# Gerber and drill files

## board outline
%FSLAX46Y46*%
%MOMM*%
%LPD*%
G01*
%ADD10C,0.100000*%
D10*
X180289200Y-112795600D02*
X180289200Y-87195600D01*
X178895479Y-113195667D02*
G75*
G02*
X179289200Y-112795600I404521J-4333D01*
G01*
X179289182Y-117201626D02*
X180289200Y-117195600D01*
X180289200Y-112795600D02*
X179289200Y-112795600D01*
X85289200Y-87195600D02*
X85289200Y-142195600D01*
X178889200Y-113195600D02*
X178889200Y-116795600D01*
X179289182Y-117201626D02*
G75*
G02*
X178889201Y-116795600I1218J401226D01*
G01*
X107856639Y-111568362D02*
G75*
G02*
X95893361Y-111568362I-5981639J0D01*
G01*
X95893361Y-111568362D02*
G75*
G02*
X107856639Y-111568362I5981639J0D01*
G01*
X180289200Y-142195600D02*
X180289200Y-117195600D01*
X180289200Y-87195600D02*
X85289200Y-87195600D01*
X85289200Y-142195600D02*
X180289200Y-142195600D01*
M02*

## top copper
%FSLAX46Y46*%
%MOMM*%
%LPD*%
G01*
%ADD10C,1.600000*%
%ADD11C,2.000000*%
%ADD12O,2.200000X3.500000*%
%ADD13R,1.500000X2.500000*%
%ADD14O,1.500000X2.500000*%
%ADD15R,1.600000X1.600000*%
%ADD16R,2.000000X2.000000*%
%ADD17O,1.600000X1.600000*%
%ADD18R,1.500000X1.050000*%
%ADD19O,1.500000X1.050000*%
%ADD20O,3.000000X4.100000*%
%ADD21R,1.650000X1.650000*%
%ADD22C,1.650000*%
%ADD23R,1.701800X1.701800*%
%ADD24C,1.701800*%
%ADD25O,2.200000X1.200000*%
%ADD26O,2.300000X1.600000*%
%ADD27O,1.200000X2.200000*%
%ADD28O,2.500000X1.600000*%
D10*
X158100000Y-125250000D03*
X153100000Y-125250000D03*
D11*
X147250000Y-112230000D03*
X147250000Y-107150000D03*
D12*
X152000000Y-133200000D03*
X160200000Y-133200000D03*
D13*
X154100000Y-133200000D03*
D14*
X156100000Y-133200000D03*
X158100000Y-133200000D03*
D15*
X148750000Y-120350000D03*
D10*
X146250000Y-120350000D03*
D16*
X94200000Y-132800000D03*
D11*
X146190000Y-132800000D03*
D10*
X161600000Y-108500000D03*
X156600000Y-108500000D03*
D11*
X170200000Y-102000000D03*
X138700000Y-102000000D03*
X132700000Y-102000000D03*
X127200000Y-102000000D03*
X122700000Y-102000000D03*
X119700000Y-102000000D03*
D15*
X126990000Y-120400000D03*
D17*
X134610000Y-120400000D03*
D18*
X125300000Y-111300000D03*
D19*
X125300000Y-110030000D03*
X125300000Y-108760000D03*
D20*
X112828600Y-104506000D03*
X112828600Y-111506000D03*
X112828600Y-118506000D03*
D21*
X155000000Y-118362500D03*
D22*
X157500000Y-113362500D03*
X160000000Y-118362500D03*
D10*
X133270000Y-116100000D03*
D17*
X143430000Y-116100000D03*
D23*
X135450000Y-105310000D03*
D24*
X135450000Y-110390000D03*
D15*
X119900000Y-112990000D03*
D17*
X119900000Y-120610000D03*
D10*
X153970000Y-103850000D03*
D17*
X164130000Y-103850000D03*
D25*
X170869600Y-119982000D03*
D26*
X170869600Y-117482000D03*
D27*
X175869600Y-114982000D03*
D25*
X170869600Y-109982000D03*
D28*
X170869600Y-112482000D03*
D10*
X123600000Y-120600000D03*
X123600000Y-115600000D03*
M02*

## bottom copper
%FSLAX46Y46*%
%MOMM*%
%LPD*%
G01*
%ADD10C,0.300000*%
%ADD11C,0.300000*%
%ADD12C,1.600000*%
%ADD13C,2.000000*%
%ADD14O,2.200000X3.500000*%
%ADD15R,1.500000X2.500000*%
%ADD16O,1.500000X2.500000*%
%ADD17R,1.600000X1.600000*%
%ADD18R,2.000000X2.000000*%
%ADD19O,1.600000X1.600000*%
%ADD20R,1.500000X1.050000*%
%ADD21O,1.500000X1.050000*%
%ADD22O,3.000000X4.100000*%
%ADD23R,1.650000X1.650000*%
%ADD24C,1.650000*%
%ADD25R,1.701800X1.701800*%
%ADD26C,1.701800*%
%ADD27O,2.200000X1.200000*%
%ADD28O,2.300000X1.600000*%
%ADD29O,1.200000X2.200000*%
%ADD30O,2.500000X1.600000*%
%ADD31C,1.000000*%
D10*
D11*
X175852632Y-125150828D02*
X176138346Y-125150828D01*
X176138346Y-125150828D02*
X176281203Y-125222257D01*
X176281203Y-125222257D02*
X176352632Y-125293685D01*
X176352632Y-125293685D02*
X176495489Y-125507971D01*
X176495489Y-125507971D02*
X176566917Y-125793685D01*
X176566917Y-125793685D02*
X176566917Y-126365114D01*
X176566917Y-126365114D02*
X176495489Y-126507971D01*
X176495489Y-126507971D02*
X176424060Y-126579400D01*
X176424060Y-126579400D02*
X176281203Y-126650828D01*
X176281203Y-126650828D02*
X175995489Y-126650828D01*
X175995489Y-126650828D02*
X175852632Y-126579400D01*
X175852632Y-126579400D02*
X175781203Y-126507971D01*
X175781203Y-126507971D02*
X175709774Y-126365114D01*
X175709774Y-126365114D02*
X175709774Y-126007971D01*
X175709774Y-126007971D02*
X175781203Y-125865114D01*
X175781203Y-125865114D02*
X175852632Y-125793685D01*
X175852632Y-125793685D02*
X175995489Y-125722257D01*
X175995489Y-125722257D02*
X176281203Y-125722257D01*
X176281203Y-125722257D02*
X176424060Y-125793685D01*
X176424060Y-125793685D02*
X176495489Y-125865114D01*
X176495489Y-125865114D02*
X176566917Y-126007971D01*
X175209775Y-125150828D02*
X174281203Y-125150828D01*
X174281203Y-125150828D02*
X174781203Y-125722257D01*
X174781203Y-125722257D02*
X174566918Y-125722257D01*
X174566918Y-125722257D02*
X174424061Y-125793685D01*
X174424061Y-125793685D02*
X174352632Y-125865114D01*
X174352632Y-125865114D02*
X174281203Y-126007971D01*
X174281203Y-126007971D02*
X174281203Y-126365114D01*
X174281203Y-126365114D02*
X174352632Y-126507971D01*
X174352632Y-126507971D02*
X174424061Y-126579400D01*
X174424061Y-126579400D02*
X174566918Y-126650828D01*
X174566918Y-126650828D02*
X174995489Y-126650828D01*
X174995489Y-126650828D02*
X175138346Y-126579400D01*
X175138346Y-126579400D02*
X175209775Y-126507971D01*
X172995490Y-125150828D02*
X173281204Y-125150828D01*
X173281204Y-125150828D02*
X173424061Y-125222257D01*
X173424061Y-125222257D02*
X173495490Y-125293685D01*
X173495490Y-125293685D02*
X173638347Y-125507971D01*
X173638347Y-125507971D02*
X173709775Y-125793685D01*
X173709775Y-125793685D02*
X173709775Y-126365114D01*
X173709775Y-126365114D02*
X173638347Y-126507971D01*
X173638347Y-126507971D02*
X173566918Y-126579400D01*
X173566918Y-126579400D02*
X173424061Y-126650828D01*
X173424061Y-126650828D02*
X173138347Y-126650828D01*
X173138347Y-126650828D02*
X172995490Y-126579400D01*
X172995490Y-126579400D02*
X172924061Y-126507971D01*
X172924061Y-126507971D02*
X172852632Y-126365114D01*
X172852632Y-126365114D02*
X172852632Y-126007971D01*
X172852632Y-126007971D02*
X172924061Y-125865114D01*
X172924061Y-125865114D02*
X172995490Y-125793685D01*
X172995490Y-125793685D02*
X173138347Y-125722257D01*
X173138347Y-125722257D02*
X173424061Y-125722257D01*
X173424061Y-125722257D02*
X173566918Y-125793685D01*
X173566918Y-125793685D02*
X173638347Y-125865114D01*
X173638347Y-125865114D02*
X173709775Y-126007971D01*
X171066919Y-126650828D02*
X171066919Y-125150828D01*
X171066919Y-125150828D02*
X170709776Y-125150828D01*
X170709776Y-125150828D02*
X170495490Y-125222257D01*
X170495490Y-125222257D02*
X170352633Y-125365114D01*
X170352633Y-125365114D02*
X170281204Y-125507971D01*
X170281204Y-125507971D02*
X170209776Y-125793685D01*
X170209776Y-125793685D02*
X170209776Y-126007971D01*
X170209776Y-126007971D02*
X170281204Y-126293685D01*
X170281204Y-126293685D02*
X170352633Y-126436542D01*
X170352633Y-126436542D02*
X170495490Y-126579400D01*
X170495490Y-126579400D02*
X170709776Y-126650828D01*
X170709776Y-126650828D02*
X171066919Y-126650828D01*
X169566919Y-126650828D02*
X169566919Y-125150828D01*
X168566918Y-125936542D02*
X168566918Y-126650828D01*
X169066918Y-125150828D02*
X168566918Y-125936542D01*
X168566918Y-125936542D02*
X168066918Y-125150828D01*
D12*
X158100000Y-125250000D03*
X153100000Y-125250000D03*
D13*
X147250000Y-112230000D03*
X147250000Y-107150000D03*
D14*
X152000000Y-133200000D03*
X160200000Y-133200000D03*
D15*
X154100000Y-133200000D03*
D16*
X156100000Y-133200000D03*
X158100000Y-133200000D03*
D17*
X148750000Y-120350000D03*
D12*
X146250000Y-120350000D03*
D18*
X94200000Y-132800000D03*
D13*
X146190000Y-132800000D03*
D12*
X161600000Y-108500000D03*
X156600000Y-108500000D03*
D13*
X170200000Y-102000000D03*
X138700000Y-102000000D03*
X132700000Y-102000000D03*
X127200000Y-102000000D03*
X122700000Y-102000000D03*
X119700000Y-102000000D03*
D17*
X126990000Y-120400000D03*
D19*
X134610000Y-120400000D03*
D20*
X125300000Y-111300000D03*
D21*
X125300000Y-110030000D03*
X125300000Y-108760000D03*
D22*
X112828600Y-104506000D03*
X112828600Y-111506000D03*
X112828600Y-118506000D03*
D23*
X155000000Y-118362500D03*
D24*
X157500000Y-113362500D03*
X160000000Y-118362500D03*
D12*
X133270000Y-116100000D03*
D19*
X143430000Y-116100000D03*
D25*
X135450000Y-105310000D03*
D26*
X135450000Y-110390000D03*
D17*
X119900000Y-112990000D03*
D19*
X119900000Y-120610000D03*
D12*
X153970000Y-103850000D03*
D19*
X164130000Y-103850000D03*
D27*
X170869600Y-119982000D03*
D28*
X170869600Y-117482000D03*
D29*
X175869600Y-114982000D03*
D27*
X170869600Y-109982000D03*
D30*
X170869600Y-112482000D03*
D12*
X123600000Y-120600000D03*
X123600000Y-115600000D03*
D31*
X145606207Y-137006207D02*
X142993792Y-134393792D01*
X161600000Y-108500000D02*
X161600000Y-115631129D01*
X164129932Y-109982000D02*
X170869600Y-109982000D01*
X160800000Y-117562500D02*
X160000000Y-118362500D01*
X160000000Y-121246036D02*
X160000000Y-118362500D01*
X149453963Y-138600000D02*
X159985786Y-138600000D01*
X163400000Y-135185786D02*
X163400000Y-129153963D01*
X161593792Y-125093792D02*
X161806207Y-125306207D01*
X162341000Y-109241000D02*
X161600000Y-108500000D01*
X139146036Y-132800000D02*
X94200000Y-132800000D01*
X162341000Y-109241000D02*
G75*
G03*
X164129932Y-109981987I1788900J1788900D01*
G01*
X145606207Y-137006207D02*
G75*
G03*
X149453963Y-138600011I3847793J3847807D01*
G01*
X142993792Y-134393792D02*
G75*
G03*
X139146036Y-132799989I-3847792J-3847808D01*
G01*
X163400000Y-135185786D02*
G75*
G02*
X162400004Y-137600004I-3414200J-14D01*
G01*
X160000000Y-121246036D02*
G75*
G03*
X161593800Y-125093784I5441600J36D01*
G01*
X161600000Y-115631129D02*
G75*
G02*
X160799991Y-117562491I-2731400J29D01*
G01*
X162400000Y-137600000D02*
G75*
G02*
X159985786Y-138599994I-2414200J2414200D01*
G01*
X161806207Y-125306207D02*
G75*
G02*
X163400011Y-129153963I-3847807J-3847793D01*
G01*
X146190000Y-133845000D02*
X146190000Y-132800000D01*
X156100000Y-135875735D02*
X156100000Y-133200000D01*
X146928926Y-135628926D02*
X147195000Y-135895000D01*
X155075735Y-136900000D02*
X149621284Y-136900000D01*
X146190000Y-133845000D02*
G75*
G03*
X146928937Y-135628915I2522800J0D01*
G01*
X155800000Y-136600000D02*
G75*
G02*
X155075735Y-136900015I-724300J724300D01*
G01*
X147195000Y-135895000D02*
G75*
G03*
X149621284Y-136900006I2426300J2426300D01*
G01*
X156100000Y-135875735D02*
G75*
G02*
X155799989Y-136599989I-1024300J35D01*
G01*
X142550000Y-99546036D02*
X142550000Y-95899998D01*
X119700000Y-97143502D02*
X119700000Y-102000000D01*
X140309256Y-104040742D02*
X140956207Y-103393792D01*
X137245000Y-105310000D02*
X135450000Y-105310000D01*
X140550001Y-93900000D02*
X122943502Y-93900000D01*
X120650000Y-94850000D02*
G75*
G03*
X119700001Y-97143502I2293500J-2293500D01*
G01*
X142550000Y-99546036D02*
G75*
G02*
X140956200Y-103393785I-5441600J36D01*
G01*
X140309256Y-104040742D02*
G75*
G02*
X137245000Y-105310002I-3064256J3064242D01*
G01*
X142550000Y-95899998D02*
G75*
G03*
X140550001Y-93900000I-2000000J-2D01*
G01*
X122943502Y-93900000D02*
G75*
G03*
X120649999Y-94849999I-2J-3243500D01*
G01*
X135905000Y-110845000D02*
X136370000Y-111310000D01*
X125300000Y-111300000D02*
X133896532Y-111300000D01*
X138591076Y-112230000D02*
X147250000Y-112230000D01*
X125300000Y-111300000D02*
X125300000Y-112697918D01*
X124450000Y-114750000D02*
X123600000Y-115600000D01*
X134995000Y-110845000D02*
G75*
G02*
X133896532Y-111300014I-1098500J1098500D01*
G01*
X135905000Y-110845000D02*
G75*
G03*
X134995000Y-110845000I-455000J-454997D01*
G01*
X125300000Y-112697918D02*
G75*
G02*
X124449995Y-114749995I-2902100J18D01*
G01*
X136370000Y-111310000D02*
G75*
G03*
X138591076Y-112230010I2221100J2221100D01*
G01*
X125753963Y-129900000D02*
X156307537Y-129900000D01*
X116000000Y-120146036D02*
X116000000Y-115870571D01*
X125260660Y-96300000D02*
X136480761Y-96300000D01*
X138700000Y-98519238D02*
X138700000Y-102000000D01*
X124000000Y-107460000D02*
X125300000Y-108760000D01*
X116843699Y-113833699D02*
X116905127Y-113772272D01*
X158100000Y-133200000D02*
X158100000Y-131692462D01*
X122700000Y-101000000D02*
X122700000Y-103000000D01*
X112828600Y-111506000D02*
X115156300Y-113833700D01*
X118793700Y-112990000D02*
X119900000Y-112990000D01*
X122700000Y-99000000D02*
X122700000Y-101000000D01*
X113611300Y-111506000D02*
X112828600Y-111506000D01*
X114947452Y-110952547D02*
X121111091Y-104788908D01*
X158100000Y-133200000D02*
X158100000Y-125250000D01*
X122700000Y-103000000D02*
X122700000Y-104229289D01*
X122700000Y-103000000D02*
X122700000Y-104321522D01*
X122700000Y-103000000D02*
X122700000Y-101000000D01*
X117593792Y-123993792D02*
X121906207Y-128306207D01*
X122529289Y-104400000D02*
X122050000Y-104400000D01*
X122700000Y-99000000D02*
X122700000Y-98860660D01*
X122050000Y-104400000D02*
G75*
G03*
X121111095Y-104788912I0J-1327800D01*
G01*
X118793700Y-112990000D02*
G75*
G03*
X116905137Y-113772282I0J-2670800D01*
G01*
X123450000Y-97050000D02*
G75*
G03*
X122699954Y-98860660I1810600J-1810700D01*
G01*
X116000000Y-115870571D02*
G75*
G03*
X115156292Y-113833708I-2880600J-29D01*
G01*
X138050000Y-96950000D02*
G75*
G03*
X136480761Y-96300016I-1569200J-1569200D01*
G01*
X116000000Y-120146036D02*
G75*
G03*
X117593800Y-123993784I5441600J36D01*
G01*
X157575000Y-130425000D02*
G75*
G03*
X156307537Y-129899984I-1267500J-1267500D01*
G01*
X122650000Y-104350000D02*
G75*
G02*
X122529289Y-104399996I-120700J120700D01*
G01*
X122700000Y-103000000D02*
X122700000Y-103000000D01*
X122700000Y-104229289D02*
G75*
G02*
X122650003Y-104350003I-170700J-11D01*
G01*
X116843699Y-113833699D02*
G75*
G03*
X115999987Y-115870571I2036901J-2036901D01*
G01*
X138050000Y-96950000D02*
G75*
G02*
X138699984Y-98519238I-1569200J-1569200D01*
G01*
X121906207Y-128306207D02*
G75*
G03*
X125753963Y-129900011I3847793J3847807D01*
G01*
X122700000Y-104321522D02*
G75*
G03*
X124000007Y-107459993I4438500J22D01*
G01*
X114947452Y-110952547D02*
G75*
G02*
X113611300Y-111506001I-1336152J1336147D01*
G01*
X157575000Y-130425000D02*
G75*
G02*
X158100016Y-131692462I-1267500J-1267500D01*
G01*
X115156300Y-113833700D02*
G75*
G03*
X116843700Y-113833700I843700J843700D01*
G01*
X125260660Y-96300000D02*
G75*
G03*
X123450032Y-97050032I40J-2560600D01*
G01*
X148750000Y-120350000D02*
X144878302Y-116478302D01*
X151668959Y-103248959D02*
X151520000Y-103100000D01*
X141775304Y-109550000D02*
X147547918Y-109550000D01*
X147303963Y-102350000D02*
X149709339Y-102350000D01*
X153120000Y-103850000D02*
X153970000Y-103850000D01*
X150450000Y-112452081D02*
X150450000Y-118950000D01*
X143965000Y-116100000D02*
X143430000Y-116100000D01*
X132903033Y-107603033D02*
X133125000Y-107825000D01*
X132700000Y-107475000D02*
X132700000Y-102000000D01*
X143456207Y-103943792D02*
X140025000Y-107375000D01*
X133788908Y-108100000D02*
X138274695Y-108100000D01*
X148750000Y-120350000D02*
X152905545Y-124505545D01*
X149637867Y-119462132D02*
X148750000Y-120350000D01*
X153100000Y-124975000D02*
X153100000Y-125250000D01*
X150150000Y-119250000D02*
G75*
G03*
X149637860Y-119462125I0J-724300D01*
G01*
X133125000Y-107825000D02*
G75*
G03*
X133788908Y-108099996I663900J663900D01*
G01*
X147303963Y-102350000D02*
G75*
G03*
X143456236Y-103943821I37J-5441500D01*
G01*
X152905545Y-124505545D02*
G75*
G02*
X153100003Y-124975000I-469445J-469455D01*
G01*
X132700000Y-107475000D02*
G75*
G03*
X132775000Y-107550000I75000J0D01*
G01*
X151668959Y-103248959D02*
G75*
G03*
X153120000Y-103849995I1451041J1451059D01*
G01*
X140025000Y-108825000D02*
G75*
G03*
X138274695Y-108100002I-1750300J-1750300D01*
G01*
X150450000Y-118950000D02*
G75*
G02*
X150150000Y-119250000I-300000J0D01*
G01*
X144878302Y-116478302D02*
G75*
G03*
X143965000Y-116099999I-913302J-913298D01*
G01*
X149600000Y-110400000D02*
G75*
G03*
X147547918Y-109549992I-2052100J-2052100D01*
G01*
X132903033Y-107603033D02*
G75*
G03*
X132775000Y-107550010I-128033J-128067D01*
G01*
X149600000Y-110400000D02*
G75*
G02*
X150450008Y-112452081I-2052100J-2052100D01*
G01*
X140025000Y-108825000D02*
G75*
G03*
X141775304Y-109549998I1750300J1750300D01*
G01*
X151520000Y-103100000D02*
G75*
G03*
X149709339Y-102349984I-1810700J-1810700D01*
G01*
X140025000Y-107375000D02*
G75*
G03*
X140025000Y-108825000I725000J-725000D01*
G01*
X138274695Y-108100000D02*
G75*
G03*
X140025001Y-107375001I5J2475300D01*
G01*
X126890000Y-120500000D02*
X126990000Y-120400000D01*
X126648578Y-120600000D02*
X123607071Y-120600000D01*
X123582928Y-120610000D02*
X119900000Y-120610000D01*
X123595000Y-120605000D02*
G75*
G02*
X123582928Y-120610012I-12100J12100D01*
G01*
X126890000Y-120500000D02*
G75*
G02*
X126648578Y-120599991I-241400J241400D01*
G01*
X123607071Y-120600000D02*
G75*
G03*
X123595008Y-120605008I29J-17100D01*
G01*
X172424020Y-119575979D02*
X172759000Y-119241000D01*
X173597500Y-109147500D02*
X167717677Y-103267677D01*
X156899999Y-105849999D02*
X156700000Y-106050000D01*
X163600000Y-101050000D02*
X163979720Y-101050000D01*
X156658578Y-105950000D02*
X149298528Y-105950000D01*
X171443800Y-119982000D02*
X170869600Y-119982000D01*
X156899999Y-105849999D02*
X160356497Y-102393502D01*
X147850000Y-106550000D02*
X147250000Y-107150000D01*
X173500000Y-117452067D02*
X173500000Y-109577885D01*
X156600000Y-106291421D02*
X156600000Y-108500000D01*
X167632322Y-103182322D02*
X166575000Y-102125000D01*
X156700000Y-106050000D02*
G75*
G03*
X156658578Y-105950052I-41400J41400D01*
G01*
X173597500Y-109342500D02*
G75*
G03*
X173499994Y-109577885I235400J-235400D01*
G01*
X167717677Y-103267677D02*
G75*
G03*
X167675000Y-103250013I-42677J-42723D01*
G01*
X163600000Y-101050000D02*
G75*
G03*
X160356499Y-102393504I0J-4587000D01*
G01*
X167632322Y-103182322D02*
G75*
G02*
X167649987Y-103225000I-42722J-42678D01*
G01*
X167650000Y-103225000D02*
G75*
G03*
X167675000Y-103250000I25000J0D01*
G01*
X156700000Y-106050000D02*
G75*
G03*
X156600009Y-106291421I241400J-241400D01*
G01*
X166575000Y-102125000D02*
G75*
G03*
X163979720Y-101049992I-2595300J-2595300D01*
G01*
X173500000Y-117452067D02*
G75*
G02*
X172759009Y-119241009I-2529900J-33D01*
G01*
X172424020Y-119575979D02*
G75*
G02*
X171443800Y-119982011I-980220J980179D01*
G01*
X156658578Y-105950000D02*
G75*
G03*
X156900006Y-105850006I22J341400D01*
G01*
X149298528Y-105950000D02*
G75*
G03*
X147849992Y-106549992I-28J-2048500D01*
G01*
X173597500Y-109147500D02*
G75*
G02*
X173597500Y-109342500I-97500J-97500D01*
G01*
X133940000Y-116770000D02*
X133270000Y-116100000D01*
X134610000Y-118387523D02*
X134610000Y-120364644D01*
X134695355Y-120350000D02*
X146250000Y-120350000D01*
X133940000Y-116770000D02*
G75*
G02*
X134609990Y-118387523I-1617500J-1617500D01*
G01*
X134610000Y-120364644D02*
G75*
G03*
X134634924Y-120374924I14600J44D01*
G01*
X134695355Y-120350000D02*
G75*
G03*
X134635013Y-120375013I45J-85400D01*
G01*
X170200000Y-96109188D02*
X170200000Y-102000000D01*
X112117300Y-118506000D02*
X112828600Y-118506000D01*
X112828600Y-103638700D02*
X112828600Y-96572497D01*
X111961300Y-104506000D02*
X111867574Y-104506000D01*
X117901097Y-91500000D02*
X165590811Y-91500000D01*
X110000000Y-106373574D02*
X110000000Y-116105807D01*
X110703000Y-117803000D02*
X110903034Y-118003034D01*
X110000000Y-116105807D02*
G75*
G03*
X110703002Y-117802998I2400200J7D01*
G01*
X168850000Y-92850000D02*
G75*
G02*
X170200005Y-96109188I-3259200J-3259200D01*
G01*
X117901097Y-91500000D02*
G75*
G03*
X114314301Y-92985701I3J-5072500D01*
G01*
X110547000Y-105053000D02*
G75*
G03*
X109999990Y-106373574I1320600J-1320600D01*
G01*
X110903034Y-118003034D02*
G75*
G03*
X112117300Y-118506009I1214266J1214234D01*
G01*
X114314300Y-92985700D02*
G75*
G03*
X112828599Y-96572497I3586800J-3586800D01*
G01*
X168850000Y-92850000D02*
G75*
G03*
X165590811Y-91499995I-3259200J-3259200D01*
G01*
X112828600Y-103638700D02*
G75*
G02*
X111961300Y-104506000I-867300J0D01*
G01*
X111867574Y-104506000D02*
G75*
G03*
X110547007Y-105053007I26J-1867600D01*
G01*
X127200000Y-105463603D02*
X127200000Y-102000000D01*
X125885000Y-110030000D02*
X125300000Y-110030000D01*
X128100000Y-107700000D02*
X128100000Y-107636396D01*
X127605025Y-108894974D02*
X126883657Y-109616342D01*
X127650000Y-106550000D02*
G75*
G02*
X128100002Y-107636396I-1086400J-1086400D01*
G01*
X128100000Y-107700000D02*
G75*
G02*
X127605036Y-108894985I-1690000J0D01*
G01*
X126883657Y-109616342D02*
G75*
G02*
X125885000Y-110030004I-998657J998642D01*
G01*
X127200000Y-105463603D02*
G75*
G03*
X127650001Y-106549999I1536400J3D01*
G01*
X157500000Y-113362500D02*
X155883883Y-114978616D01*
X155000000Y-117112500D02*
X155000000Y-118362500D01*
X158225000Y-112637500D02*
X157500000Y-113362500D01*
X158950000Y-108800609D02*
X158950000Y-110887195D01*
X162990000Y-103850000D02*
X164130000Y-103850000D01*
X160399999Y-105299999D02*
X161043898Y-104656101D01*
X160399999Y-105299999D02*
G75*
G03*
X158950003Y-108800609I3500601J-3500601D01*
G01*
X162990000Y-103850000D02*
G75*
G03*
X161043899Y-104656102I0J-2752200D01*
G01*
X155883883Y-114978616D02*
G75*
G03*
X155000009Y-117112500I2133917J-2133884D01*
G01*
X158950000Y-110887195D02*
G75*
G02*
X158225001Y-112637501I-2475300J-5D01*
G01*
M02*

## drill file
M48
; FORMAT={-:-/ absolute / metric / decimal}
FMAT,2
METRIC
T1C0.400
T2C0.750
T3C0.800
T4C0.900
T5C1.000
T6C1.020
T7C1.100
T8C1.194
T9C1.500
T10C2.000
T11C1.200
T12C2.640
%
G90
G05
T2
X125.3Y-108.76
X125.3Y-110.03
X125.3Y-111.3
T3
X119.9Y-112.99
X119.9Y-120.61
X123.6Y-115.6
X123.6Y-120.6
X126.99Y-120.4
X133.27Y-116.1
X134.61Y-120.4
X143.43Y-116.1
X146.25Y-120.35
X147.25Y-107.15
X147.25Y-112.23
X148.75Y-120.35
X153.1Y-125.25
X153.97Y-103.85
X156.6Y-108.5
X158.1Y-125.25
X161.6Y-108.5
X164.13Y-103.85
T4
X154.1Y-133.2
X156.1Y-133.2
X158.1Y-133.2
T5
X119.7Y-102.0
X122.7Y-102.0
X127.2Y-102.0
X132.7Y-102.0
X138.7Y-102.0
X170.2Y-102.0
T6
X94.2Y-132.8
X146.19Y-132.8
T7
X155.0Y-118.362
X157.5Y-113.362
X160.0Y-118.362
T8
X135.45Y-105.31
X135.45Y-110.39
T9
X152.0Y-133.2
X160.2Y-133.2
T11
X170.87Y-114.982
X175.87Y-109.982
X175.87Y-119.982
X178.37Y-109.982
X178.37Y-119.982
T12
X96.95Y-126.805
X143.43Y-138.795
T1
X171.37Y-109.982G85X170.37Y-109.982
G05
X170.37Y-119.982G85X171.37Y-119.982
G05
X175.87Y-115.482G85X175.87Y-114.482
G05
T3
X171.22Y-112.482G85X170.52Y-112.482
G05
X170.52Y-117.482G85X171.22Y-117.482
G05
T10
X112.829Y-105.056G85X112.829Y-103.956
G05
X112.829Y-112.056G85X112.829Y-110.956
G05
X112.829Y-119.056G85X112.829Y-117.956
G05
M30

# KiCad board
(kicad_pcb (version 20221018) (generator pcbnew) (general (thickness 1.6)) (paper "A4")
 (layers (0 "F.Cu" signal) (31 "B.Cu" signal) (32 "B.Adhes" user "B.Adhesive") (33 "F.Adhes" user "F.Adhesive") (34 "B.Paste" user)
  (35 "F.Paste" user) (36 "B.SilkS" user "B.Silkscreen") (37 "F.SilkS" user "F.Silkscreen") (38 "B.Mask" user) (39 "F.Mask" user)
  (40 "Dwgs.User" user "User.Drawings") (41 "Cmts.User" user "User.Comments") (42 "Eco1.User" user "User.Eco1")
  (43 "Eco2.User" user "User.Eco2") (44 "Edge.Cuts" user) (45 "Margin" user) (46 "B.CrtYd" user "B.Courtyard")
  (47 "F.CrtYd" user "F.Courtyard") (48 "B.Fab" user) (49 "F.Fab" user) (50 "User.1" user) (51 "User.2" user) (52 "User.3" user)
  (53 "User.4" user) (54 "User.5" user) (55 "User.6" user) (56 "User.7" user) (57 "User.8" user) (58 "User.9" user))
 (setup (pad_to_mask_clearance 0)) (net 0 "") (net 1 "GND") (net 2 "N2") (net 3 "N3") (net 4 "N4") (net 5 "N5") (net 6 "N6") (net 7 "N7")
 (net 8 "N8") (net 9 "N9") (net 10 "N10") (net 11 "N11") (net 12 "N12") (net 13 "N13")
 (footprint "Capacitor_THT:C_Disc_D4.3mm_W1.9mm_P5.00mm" (layer "F.Cu") (at 158.1 125.25 180)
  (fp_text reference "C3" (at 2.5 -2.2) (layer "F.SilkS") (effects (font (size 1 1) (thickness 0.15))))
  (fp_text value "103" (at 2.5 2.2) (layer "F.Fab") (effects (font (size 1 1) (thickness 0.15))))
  (pad "1" thru_hole circle (at 0 0 180) (size 1.6 1.6) (drill 0.8) (layers "*.Cu" "*.Mask") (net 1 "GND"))
  (pad "2" thru_hole circle (at 5 0 180) (size 1.6 1.6) (drill 0.8) (layers "*.Cu" "*.Mask") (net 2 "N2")))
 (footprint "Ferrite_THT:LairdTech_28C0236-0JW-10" (layer "F.Cu") (at 147.25 112.23 90)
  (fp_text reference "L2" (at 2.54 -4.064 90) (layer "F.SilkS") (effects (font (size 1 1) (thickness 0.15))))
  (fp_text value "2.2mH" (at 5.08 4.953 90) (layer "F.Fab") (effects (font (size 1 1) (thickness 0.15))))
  (pad "1" thru_hole circle (at 0 0 90) (size 2 2) (drill 0.8) (layers "*.Cu" "*.Mask") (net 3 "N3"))
  (pad "2" thru_hole circle (at 5.08 0 90) (size 2 2) (drill 0.8) (layers "*.Cu" "*.Mask") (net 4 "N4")))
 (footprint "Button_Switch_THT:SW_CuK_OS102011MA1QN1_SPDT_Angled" (layer "F.Cu") (at 154.1 133.2)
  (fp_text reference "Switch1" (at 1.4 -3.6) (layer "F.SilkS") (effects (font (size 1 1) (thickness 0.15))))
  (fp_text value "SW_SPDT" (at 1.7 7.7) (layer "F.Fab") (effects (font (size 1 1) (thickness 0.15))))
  (pad "" thru_hole oval (at -2.1 0) (size 2.2 3.5) (drill 1.5) (layers "*.Cu" "*.Mask"))
  (pad "" thru_hole oval (at 6.1 0) (size 2.2 3.5) (drill 1.5) (layers "*.Cu" "*.Mask"))
  (pad "1" thru_hole rect (at 0 0) (size 1.5 2.5) (drill 0.9) (layers "*.Cu" "*.Mask") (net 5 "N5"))
  (pad "2" thru_hole oval (at 2 0) (size 1.5 2.5) (drill 0.9) (layers "*.Cu" "*.Mask") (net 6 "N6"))
  (pad "3" thru_hole oval (at 4 0) (size 1.5 2.5) (drill 0.9) (layers "*.Cu" "*.Mask") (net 1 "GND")))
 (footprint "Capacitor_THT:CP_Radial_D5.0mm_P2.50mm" (layer "F.Cu") (at 148.75 120.35 180)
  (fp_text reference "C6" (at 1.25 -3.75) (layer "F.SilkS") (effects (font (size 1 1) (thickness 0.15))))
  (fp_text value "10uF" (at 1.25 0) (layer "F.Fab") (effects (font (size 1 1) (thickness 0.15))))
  (pad "1" thru_hole rect (at 0 0 180) (size 1.6 1.6) (drill 0.8) (layers "*.Cu" "*.Mask") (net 2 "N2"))
  (pad "2" thru_hole circle (at 2.5 0 180) (size 1.6 1.6) (drill 0.8) (layers "*.Cu" "*.Mask") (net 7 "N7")))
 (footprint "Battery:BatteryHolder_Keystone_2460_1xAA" (layer "F.Cu") (at 94.2 132.8)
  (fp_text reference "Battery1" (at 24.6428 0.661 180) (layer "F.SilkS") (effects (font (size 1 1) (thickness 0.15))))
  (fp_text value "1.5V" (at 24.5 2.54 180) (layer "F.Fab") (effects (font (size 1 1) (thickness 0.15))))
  (pad "" np_thru_hole circle (at 2.75 -5.995 90) (size 2.64 2.64) (drill 2.64) (layers "*.Cu" "*.Mask"))
  (pad "" np_thru_hole circle (at 49.23 5.995) (size 2.64 2.64) (drill 2.64) (layers "*.Cu" "*.Mask"))
  (pad "1" thru_hole rect (at 0 0 180) (size 2 2) (drill 1.02) (layers "*.Cu" "*.Mask") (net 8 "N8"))
  (pad "2" thru_hole circle (at 51.99 0 180) (size 2 2) (drill 1.02) (layers "*.Cu" "*.Mask") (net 6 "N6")))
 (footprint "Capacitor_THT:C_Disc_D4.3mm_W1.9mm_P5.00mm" (layer "F.Cu") (at 161.6 108.5 180)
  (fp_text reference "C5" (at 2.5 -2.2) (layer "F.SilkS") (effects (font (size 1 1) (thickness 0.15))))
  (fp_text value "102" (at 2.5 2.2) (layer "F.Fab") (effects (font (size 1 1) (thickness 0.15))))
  (pad "1" thru_hole circle (at 0 0 180) (size 1.6 1.6) (drill 0.8) (layers "*.Cu" "*.Mask") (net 8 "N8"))
  (pad "2" thru_hole circle (at 5 0 180) (size 1.6 1.6) (drill 0.8) (layers "*.Cu" "*.Mask") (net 4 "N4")))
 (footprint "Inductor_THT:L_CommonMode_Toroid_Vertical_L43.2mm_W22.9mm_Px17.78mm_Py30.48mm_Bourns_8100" (layer "F.Cu") (at 132.7 94.5)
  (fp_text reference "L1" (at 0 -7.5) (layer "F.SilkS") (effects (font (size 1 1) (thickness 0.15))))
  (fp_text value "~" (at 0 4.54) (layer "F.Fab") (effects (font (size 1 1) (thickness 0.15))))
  (pad "1" thru_hole circle (at 37.5 7.5) (size 2 2) (drill 1) (layers "*.Cu" "*.Mask") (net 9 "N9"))
  (pad "2" thru_hole circle (at 6 7.5) (size 2 2) (drill 1) (layers "*.Cu" "*.Mask") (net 1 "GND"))
  (pad "3" thru_hole circle (at 0 7.5) (size 2 2) (drill 1) (layers "*.Cu" "*.Mask") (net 2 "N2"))
  (pad "4" thru_hole circle (at -5.5 7.5) (size 2 2) (drill 1) (layers "*.Cu" "*.Mask") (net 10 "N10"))
  (pad "5" thru_hole circle (at -10 7.5) (size 2 2) (drill 1) (layers "*.Cu" "*.Mask") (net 1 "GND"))
  (pad "6" thru_hole circle (at -13 7.5) (size 2 2) (drill 1) (layers "*.Cu" "*.Mask") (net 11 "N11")))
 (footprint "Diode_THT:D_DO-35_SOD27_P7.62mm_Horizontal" (layer "F.Cu") (at 126.99 120.4)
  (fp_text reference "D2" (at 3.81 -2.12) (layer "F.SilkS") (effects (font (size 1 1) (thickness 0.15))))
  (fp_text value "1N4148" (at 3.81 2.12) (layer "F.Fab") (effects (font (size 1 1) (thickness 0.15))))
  (pad "1" thru_hole rect (at 0 0) (size 1.6 1.6) (drill 0.8) (layers "*.Cu" "*.Mask") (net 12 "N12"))
  (pad "2" thru_hole oval (at 7.62 0) (size 1.6 1.6) (drill 0.8) (layers "*.Cu" "*.Mask") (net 7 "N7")))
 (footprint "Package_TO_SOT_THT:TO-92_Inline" (layer "F.Cu") (at 125.3 111.3 90)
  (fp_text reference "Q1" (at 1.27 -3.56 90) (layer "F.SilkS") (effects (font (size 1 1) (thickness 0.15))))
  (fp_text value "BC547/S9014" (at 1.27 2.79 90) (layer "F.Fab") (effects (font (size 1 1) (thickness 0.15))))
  (pad "1" thru_hole rect (at 0 0 90) (size 1.05 1.5) (drill 0.75) (layers "*.Cu" "*.Mask") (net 3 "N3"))
  (pad "2" thru_hole oval (at 1.27 0 90) (size 1.05 1.5) (drill 0.75) (layers "*.Cu" "*.Mask") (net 10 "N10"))
  (pad "3" thru_hole oval (at 2.54 0 90) (size 1.05 1.5) (drill 0.75) (layers "*.Cu" "*.Mask") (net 1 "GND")))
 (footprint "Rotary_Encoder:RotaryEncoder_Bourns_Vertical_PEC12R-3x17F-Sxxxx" (layer "F.Cu") (at 101.8286 111.506)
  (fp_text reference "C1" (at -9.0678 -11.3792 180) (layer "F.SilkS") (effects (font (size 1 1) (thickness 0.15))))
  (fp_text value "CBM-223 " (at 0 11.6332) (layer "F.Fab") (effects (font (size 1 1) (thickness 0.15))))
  (pad "1" thru_hole oval (at 11 -7 90) (size 4.1 3) (drill oval 3.1 2) (layers "*.Cu" "*.Mask") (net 9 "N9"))
  (pad "2" thru_hole oval (at 11 0 90) (size 4.1 3) (drill oval 3.1 2) (layers "*.Cu" "*.Mask") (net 1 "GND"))
  (pad "3" thru_hole oval (at 11 7 90) (size 4.1 3) (drill oval 3.1 2) (layers "*.Cu" "*.Mask") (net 9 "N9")))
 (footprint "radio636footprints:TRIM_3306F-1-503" (layer "F.Cu") (at 157.5 115.8625 -90)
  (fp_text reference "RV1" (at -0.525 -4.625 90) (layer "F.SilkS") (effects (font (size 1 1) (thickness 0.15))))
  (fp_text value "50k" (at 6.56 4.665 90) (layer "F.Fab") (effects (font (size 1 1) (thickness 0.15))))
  (pad "1" thru_hole rect (at 2.5 2.5 270) (size 1.65 1.65) (drill 1.1) (layers "*.Cu" "*.Mask") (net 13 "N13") (solder_mask_margin 0.102))
  (pad "2" thru_hole circle (at -2.5 0 270) (size 1.65 1.65) (drill 1.1) (layers "*.Cu" "*.Mask") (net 13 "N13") (solder_mask_margin 0.102))
  (pad "3" thru_hole circle (at 2.5 -2.5 270) (size 1.65 1.65) (drill 1.1) (layers "*.Cu" "*.Mask") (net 8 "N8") (solder_mask_margin 0.102)))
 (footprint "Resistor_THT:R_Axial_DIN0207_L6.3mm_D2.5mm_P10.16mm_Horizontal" (layer "F.Cu") (at 133.27 116.1)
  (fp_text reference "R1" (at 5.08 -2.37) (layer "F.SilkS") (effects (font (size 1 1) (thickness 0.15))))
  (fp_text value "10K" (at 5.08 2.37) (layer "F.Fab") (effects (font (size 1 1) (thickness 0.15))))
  (pad "1" thru_hole circle (at 0 0) (size 1.6 1.6) (drill 0.8) (layers "*.Cu" "*.Mask") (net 7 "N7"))
  (pad "2" thru_hole oval (at 10.16 0) (size 1.6 1.6) (drill 0.8) (layers "*.Cu" "*.Mask") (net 2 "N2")))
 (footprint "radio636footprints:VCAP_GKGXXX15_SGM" (layer "F.Cu") (at 135.45 105.31 -90)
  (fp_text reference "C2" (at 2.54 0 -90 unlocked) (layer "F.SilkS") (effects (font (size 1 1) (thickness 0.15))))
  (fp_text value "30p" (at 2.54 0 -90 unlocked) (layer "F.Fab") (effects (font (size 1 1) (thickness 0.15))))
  (pad "1" thru_hole rect (at 0 0 270) (size 1.7018 1.7018) (drill 1.1938) (layers "*.Cu" "*.Mask") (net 11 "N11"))
  (pad "2" thru_hole circle (at 5.08 0 270) (size 1.7018 1.7018) (drill 1.1938) (layers "*.Cu" "*.Mask") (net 3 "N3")))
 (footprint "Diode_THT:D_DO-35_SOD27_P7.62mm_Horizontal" (layer "F.Cu") (at 119.9 112.99 -90)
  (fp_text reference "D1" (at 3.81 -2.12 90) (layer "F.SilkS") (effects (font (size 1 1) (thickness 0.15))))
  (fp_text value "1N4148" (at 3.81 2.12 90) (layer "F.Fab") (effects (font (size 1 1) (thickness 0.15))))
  (pad "1" thru_hole rect (at 0 0 270) (size 1.6 1.6) (drill 0.8) (layers "*.Cu" "*.Mask") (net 1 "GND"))
  (pad "2" thru_hole oval (at 7.62 0 270) (size 1.6 1.6) (drill 0.8) (layers "*.Cu" "*.Mask") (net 12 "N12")))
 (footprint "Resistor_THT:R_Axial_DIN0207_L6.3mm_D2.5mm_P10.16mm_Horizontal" (layer "F.Cu") (at 153.97 103.85)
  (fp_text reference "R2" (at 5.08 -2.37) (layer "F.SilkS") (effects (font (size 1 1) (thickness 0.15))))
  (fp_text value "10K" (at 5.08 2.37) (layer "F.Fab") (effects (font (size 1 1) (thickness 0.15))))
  (pad "1" thru_hole circle (at 0 0) (size 1.6 1.6) (drill 0.8) (layers "*.Cu" "*.Mask") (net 2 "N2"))
  (pad "2" thru_hole oval (at 10.16 0) (size 1.6 1.6) (drill 0.8) (layers "*.Cu" "*.Mask") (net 13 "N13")))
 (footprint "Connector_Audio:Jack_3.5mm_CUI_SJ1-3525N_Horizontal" (layer "F.Cu") (at 175.8696 114.982 90)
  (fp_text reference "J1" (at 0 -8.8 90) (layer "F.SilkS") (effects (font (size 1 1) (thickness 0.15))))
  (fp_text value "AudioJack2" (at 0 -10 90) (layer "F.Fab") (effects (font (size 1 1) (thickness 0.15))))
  (pad "" np_thru_hole circle (at -5 0 90) (size 1.2 1.2) (drill 1.2) (layers "F&B.Cu" "*.Mask"))
  (pad "" np_thru_hole circle (at -5 2.5 90) (size 1.2 1.2) (drill 1.2) (layers "F&B.Cu" "*.Mask"))
  (pad "" np_thru_hole circle (at 0 -5 90) (size 1.2 1.2) (drill 1.2) (layers "F&B.Cu" "*.Mask"))
  (pad "" np_thru_hole circle (at 5 0 90) (size 1.2 1.2) (drill 1.2) (layers "F&B.Cu" "*.Mask"))
  (pad "" np_thru_hole circle (at 5 2.5 90) (size 1.2 1.2) (drill 1.2) (layers "F&B.Cu" "*.Mask"))
  (pad "R" thru_hole oval (at -5 -5 90) (size 1.2 2.2) (drill oval 0.4 1.4) (layers "*.Cu" "*.Mask") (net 4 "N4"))
  (pad "RN" thru_hole oval (at -2.5 -5 90) (size 1.6 2.3) (drill oval 0.8 1.5) (layers "*.Cu" "*.Mask"))
  (pad "S" thru_hole oval (at 0 0 90) (size 2.2 1.2) (drill oval 1.4 0.4) (layers "*.Cu" "*.Mask"))
  (pad "T" thru_hole oval (at 5 -5 270) (size 1.2 2.2) (drill oval 0.4 1.4) (layers "*.Cu" "*.Mask") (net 8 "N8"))
  (pad "TN" thru_hole oval (at 2.5 -5 270) (size 1.6 2.5) (drill oval 0.8 1.5) (layers "*.Cu" "*.Mask")))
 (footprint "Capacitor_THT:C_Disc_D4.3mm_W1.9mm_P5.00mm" (layer "F.Cu") (at 123.6 120.6 90)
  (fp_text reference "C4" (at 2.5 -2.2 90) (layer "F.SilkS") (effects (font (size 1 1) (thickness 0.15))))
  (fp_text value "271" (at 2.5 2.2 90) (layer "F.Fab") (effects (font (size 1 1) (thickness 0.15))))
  (pad "1" thru_hole circle (at 0 0 90) (size 1.6 1.6) (drill 0.8) (layers "*.Cu" "*.Mask") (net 12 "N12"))
  (pad "2" thru_hole circle (at 5 0 90) (size 1.6 1.6) (drill 0.8) (layers "*.Cu" "*.Mask") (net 3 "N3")))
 (gr_line (start 180.2892 112.7956) (end 180.2892 87.1956) (stroke (width 0.1) (type default)) (layer "Edge.Cuts"))
 (gr_arc (start 178.895479 113.195667) (mid 179.011666 112.91624) (end 179.2892 112.7956) (stroke (width 0.1) (type default))
  (layer "Edge.Cuts"))
 (gr_line (start 179.289182 117.201626) (end 180.2892 117.1956) (stroke (width 0.1) (type default)) (layer "Edge.Cuts"))
 (gr_line (start 180.2892 112.7956) (end 179.2892 112.7956) (stroke (width 0.1) (type default)) (layer "Edge.Cuts"))
 (gr_line (start 85.2892 87.1956) (end 85.2892 142.1956) (stroke (width 0.1) (type default)) (layer "Edge.Cuts"))
 (gr_line (start 178.8892 113.1956) (end 178.8892 116.7956) (stroke (width 0.1) (type default)) (layer "Edge.Cuts"))
 (gr_arc (start 179.289182 117.201626) (mid 179.004569 117.081975) (end 178.889201 116.7956) (stroke (width 0.1) (type default))
  (layer "Edge.Cuts"))
 (gr_circle (center 101.875 111.568362) (end 106.575 115.268362) (stroke (width 0.1) (type default)) (fill none) (layer "Edge.Cuts"))
 (gr_line (start 180.2892 142.1956) (end 180.2892 117.1956) (stroke (width 0.1) (type default)) (layer "Edge.Cuts"))
 (gr_line (start 180.2892 87.1956) (end 85.2892 87.1956) (stroke (width 0.1) (type default)) (layer "Edge.Cuts"))
 (gr_line (start 85.2892 142.1956) (end 180.2892 142.1956) (stroke (width 0.1) (type default)) (layer "Edge.Cuts"))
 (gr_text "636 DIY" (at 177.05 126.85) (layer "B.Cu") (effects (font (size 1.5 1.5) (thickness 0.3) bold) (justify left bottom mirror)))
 (segment (start 145.606207 137.006207) (end 142.993792 134.393792) (width 1) (layer "B.Cu") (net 8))
 (segment (start 161.6 108.5) (end 161.6 115.631129) (width 1) (layer "B.Cu") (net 8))
 (segment (start 164.129932 109.982) (end 170.8696 109.982) (width 1) (layer "B.Cu") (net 8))
 (segment (start 160.8 117.5625) (end 160 118.3625) (width 1) (layer "B.Cu") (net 8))
 (segment (start 160 121.246036) (end 160 118.3625) (width 1) (layer "B.Cu") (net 8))
 (segment (start 149.453963 138.6) (end 159.985786 138.6) (width 1) (layer "B.Cu") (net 8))
 (segment (start 163.4 135.185786) (end 163.4 129.153963) (width 1) (layer "B.Cu") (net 8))
 (segment (start 161.593792 125.093792) (end 161.806207 125.306207) (width 1) (layer "B.Cu") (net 8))
 (segment (start 162.341 109.241) (end 161.6 108.5) (width 1) (layer "B.Cu") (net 8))
 (segment (start 139.146036 132.8) (end 94.2 132.8) (width 1) (layer "B.Cu") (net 8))
 (arc (start 162.341 109.241) (mid 163.161769 109.78942) (end 164.129932 109.982) (width 1) (layer "B.Cu") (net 8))
 (arc (start 145.606207 137.006207) (mid 147.371572 138.185786) (end 149.453963 138.6) (width 1) (layer "B.Cu") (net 8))
 (arc (start 142.993792 134.393792) (mid 141.228426 133.214213) (end 139.146036 132.8) (width 1) (layer "B.Cu") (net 8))
 (arc (start 163.4 135.185786) (mid 163.140108 136.492349) (end 162.4 137.6) (width 1) (layer "B.Cu") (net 8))
 (arc (start 160 121.246036) (mid 160.414213 123.328426) (end 161.593792 125.093792) (width 1) (layer "B.Cu") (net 8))
 (arc (start 161.6 115.631129) (mid 161.392086 116.676379) (end 160.8 117.5625) (width 1) (layer "B.Cu") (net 8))
 (arc (start 162.4 137.6) (mid 161.292349 138.340108) (end 159.985786 138.6) (width 1) (layer "B.Cu") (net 8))
 (arc (start 161.806207 125.306207) (mid 162.985786 127.071572) (end 163.4 129.153963) (width 1) (layer "B.Cu") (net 8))
 (segment (start 146.19 133.845) (end 146.19 132.8) (width 1) (layer "B.Cu") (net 6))
 (segment (start 156.1 135.875735) (end 156.1 133.2) (width 1) (layer "B.Cu") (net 6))
 (segment (start 146.928926 135.628926) (end 147.195 135.895) (width 1) (layer "B.Cu") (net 6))
 (segment (start 155.075735 136.9) (end 149.621284 136.9) (width 1) (layer "B.Cu") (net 6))
 (arc (start 146.19 133.845) (mid 146.38204 134.810453) (end 146.928926 135.628926) (width 1) (layer "B.Cu") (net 6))
 (arc (start 155.8 136.6) (mid 155.467704 136.822032) (end 155.075735 136.9) (width 1) (layer "B.Cu") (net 6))
 (arc (start 147.195 135.895) (mid 148.308188 136.638809) (end 149.621284 136.9) (width 1) (layer "B.Cu") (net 6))
 (arc (start 156.1 135.875735) (mid 156.022032 136.267704) (end 155.8 136.6) (width 1) (layer "B.Cu") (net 6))
 (segment (start 142.55 99.546036) (end 142.55 95.899998) (width 1) (layer "B.Cu") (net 11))
 (segment (start 119.7 97.143502) (end 119.7 102) (width 1) (layer "B.Cu") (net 11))
 (segment (start 140.309256 104.040742) (end 140.956207 103.393792) (width 1) (layer "B.Cu") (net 11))
 (segment (start 137.245 105.31) (end 135.45 105.31) (width 1) (layer "B.Cu") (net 11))
 (segment (start 140.550001 93.9) (end 122.943502 93.9) (width 1) (layer "B.Cu") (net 11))
 (arc (start 120.65 94.85) (mid 119.946896 95.902267) (end 119.7 97.143502) (width 1) (layer "B.Cu") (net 11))
 (arc (start 142.55 99.546036) (mid 142.135786 101.628426) (end 140.956207 103.393792) (width 1) (layer "B.Cu") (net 11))
 (arc (start 140.309256 104.040742) (mid 138.903363 104.98013) (end 137.245 105.31) (width 1) (layer "B.Cu") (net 11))
 (arc (start 142.55 95.899998) (mid 141.964213 94.485785) (end 140.550001 93.9) (width 1) (layer "B.Cu") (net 11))
 (arc (start 122.943502 93.9) (mid 121.702267 94.146896) (end 120.65 94.85) (width 1) (layer "B.Cu") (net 11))
 (segment (start 135.905 110.845) (end 136.37 111.31) (width 1) (layer "B.Cu") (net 3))
 (segment (start 125.3 111.3) (end 133.896532 111.3) (width 1) (layer "B.Cu") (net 3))
 (segment (start 138.591076 112.23) (end 147.25 112.23) (width 1) (layer "B.Cu") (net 3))
 (segment (start 125.3 111.3) (end 125.3 112.697918) (width 1) (layer "B.Cu") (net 3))
 (segment (start 124.45 114.75) (end 123.6 115.6) (width 1) (layer "B.Cu") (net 3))
 (arc (start 134.995 110.845) (mid 134.491018 111.181749) (end 133.896532 111.3) (width 1) (layer "B.Cu") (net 3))
 (arc (start 135.905 110.845) (mid 135.45 110.656532) (end 134.995 110.845) (width 1) (layer "B.Cu") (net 3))
 (arc (start 125.3 112.697918) (mid 125.079092 113.808496) (end 124.45 114.75) (width 1) (layer "B.Cu") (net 3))
 (arc (start 136.37 111.31) (mid 137.389038 111.990899) (end 138.591076 112.23) (width 1) (layer "B.Cu") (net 3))
 (segment (start 125.753963 129.9) (end 156.307537 129.9) (width 1) (layer "B.Cu") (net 1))
 (segment (start 116 120.146036) (end 116 115.870571) (width 1) (layer "B.Cu") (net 1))
 (segment (start 125.26066 96.3) (end 136.480761 96.3) (width 1) (layer "B.Cu") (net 1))
 (segment (start 138.7 98.519238) (end 138.7 102) (width 1) (layer "B.Cu") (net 1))
 (segment (start 124 107.46) (end 125.3 108.76) (width 1) (layer "B.Cu") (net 1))
 (segment (start 116.843699 113.833699) (end 116.905127 113.772272) (width 1) (layer "B.Cu") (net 1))
 (segment (start 158.1 133.2) (end 158.1 131.692462) (width 1) (layer "B.Cu") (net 1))
 (segment (start 122.7 101) (end 122.7 103) (width 1) (layer "B.Cu") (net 1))
 (segment (start 112.8286 111.506) (end 115.1563 113.8337) (width 1) (layer "B.Cu") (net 1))
 (segment (start 118.7937 112.99) (end 119.9 112.99) (width 1) (layer "B.Cu") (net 1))
 (segment (start 122.7 99) (end 122.7 101) (width 1) (layer "B.Cu") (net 1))
 (segment (start 113.6113 111.506) (end 112.8286 111.506) (width 1) (layer "B.Cu") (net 1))
 (segment (start 114.947452 110.952547) (end 121.111091 104.788908) (width 1) (layer "B.Cu") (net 1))
 (segment (start 158.1 133.2) (end 158.1 125.25) (width 1) (layer "B.Cu") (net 1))
 (segment (start 122.7 103) (end 122.7 104.229289) (width 1) (layer "B.Cu") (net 1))
 (segment (start 122.7 103) (end 122.7 104.321522) (width 1) (layer "B.Cu") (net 1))
 (segment (start 122.7 103) (end 122.7 101) (width 1) (layer "B.Cu") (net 1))
 (segment (start 117.593792 123.993792) (end 121.906207 128.306207) (width 1) (layer "B.Cu") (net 1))
 (segment (start 122.529289 104.4) (end 122.05 104.4) (width 1) (layer "B.Cu") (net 1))
 (segment (start 122.7 99) (end 122.7 98.86066) (width 1) (layer "B.Cu") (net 1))
 (arc (start 122.05 104.4) (mid 121.541866 104.501073) (end 121.111091 104.788908) (width 1) (layer "B.Cu") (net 1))
 (arc (start 118.7937 112.99) (mid 117.771611 113.193305) (end 116.905127 113.772272) (width 1) (layer "B.Cu") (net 1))
 (arc (start 123.45 97.05) (mid 122.894918 97.880737) (end 122.7 98.86066) (width 1) (layer "B.Cu") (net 1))
 (arc (start 116 115.870571) (mid 115.780729 114.768224) (end 115.1563 113.8337) (width 1) (layer "B.Cu") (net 1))
 (arc (start 138.05 96.95) (mid 137.330027 96.468929) (end 136.480761 96.3) (width 1) (layer "B.Cu") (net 1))
 (arc (start 116 120.146036) (mid 116.414213 122.228426) (end 117.593792 123.993792) (width 1) (layer "B.Cu") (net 1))
 (arc (start 157.575 130.425) (mid 156.993483 130.036443) (end 156.307537 129.9) (width 1) (layer "B.Cu") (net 1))
 (arc (start 122.65 104.35) (mid 122.594617 104.387005) (end 122.529289 104.4) (width 1) (layer "B.Cu") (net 1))
 (arc (start 122.7 103) (mid 122.7 103) (end 122.7 103) (width 1) (layer "B.Cu") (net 1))
 (arc (start 122.7 104.229289) (mid 122.687005 104.294617) (end 122.65 104.35) (width 1) (layer "B.Cu") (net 1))
 (arc (start 116.843699 113.833699) (mid 116.21927 114.768224) (end 116 115.870571) (width 1) (layer "B.Cu") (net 1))
 (arc (start 138.05 96.95) (mid 138.53107 97.669972) (end 138.7 98.519238) (width 1) (layer "B.Cu") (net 1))
 (arc (start 121.906207 128.306207) (mid 123.671572 129.485786) (end 125.753963 129.9) (width 1) (layer "B.Cu") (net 1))
 (arc (start 122.7 104.321522) (mid 123.037858 106.020054) (end 124 107.46) (width 1) (layer "B.Cu") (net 1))
 (arc (start 114.947452 110.952547) (mid 114.33442 111.362162) (end 113.6113 111.506) (width 1) (layer "B.Cu") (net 1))
 (arc (start 157.575 130.425) (mid 157.963556 131.006516) (end 158.1 131.692462) (width 1) (layer "B.Cu") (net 1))
 (arc (start 115.1563 113.8337) (mid 115.999999 114.183171) (end 116.843699 113.833699) (width 1) (layer "B.Cu") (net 1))
 (arc (start 125.26066 96.3) (mid 124.280737 96.494918) (end 123.45 97.05) (width 1) (layer "B.Cu") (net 1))
 (segment (start 148.75 120.35) (end 144.878302 116.478302) (width 1) (layer "B.Cu") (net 2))
 (segment (start 151.668959 103.248959) (end 151.52 103.1) (width 1) (layer "B.Cu") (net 2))
 (segment (start 141.775304 109.55) (end 147.547918 109.55) (width 1) (layer "B.Cu") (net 2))
 (segment (start 147.303963 102.35) (end 149.709339 102.35) (width 1) (layer "B.Cu") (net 2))
 (segment (start 153.12 103.85) (end 153.97 103.85) (width 1) (layer "B.Cu") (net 2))
 (segment (start 150.45 112.452081) (end 150.45 118.95) (width 1) (layer "B.Cu") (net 2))
 (segment (start 143.965 116.1) (end 143.43 116.1) (width 1) (layer "B.Cu") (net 2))
 (segment (start 132.903033 107.603033) (end 133.125 107.825) (width 1) (layer "B.Cu") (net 2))
 (segment (start 132.7 107.475) (end 132.7 102) (width 1) (layer "B.Cu") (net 2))
 (segment (start 143.456207 103.943792) (end 140.025 107.375) (width 1) (layer "B.Cu") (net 2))
 (segment (start 133.788908 108.1) (end 138.274695 108.1) (width 1) (layer "B.Cu") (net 2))
 (segment (start 148.75 120.35) (end 152.905545 124.505545) (width 1) (layer "B.Cu") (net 2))
 (segment (start 149.637867 119.462132) (end 148.75 120.35) (width 1) (layer "B.Cu") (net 2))
 (segment (start 153.1 124.975) (end 153.1 125.25) (width 1) (layer "B.Cu") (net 2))
 (arc (start 150.15 119.25) (mid 149.872835 119.305131) (end 149.637867 119.462132) (width 1) (layer "B.Cu") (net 2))
 (arc (start 133.125 107.825) (mid 133.429603 108.028529) (end 133.788908 108.1) (width 1) (layer "B.Cu") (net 2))
 (arc (start 147.303963 102.35) (mid 145.221572 102.764213) (end 143.456207 103.943792) (width 1) (layer "B.Cu") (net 2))
 (arc (start 152.905545 124.505545) (mid 153.049462 124.720932) (end 153.1 124.975) (width 1) (layer "B.Cu") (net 2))
 (arc (start 132.7 107.475) (mid 132.721966 107.528033) (end 132.775 107.55) (width 1) (layer "B.Cu") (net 2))
 (arc (start 151.668959 103.248959) (mid 152.334702 103.693794) (end 153.12 103.85) (width 1) (layer "B.Cu") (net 2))
 (arc (start 140.025 108.825) (mid 139.221953 108.288421) (end 138.274695 108.1) (width 1) (layer "B.Cu") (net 2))
 (arc (start 150.45 118.95) (mid 150.362132 119.162132) (end 150.15 119.25) (width 1) (layer "B.Cu") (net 2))
 (arc (start 144.878302 116.478302) (mid 144.459275 116.198317) (end 143.965 116.1) (width 1) (layer "B.Cu") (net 2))
 (arc (start 149.6 110.4) (mid 148.658496 109.770907) (end 147.547918 109.55) (width 1) (layer "B.Cu") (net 2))
 (arc (start 132.903033 107.603033) (mid 132.84429 107.563782) (end 132.775 107.55) (width 1) (layer "B.Cu") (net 2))
 (arc (start 149.6 110.4) (mid 150.229092 111.341502) (end 150.45 112.452081) (width 1) (layer "B.Cu") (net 2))
 (arc (start 140.025 108.825) (mid 140.828046 109.361578) (end 141.775304 109.55) (width 1) (layer "B.Cu") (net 2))
 (arc (start 151.52 103.1) (mid 150.689261 102.544918) (end 149.709339 102.35) (width 1) (layer "B.Cu") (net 2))
 (arc (start 140.025 107.375) (mid 139.724695 108.1) (end 140.025 108.825) (width 1) (layer "B.Cu") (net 2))
 (arc (start 138.274695 108.1) (mid 139.221953 107.911578) (end 140.025 107.375) (width 1) (layer "B.Cu") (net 2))
 (segment (start 126.89 120.5) (end 126.99 120.4) (width 1) (layer "B.Cu") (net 12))
 (segment (start 126.648578 120.6) (end 123.607071 120.6) (width 1) (layer "B.Cu") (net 12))
 (segment (start 123.582928 120.61) (end 119.9 120.61) (width 1) (layer "B.Cu") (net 12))
 (arc (start 123.595 120.605) (mid 123.589461 120.6087) (end 123.582928 120.61) (width 1) (layer "B.Cu") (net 12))
 (arc (start 126.89 120.5) (mid 126.779234 120.57401) (end 126.648578 120.6) (width 1) (layer "B.Cu") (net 12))
 (arc (start 123.607071 120.6) (mid 123.600538 120.601299) (end 123.595 120.605) (width 1) (layer "B.Cu") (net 12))
 (segment (start 172.42402 119.575979) (end 172.759 119.241) (width 1) (layer "B.Cu") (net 4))
 (segment (start 173.5975 109.1475) (end 167.717677 103.267677) (width 1) (layer "B.Cu") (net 4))
 (segment (start 156.899999 105.849999) (end 156.7 106.05) (width 1) (layer "B.Cu") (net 4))
 (segment (start 163.6 101.05) (end 163.97972 101.05) (width 1) (layer "B.Cu") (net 4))
 (segment (start 156.658578 105.95) (end 149.298528 105.95) (width 1) (layer "B.Cu") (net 4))
 (segment (start 171.4438 119.982) (end 170.8696 119.982) (width 1) (layer "B.Cu") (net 4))
 (segment (start 156.899999 105.849999) (end 160.356497 102.393502) (width 1) (layer "B.Cu") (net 4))
 (segment (start 147.85 106.55) (end 147.25 107.15) (width 1) (layer "B.Cu") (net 4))
 (segment (start 173.5 117.452067) (end 173.5 109.577885) (width 1) (layer "B.Cu") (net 4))
 (segment (start 156.6 106.291421) (end 156.6 108.5) (width 1) (layer "B.Cu") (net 4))
 (segment (start 167.632322 103.182322) (end 166.575 102.125) (width 1) (layer "B.Cu") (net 4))
 (arc (start 156.7 106.05) (mid 156.712698 105.986161) (end 156.658578 105.95) (width 1) (layer "B.Cu") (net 4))
 (arc (start 173.5975 109.3425) (mid 173.525339 109.450495) (end 173.5 109.577885) (width 1) (layer "B.Cu") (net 4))
 (arc (start 167.717677 103.267677) (mid 167.698096 103.254594) (end 167.675 103.25) (width 1) (layer "B.Cu") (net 4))
 (arc (start 163.6 101.05) (mid 161.844628 101.399164) (end 160.356497 102.393502) (width 1) (layer "B.Cu") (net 4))
 (arc (start 167.632322 103.182322) (mid 167.645405 103.201902) (end 167.65 103.225) (width 1) (layer "B.Cu") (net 4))
 (arc (start 167.65 103.225) (mid 167.657322 103.242677) (end 167.675 103.25) (width 1) (layer "B.Cu") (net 4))
 (arc (start 156.7 106.05) (mid 156.625989 106.160764) (end 156.6 106.291421) (width 1) (layer "B.Cu") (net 4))
 (arc (start 166.575 102.125) (mid 165.384275 101.329383) (end 163.97972 101.05) (width 1) (layer "B.Cu") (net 4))
 (arc (start 173.5 117.452067) (mid 173.30742 118.42023) (end 172.759 119.241) (width 1) (layer "B.Cu") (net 4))
 (arc (start 172.42402 119.575979) (mid 171.974291 119.876478) (end 171.4438 119.982) (width 1) (layer "B.Cu") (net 4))
 (arc (start 156.658578 105.95) (mid 156.789234 105.92401) (end 156.899999 105.849999) (width 1) (layer "B.Cu") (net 4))
 (arc (start 149.298528 105.95) (mid 148.51459 106.105934) (end 147.85 106.55) (width 1) (layer "B.Cu") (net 4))
 (arc (start 173.5975 109.1475) (mid 173.637885 109.245) (end 173.5975 109.3425) (width 1) (layer "B.Cu") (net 4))
 (segment (start 133.94 116.77) (end 133.27 116.1) (width 1) (layer "B.Cu") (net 7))
 (segment (start 134.61 118.387523) (end 134.61 120.364644) (width 1) (layer "B.Cu") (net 7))
 (segment (start 134.695355 120.35) (end 146.25 120.35) (width 1) (layer "B.Cu") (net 7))
 (arc (start 133.94 116.77) (mid 134.435872 117.512125) (end 134.61 118.387523) (width 1) (layer "B.Cu") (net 7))
 (arc (start 134.61 120.364644) (mid 134.61904 120.378174) (end 134.635 120.375) (width 1) (layer "B.Cu") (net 7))
 (arc (start 134.695355 120.35) (mid 134.662691 120.356497) (end 134.635 120.375) (width 1) (layer "B.Cu") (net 7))
 (segment (start 170.2 96.109188) (end 170.2 102) (width 1) (layer "B.Cu") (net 9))
 (segment (start 112.1173 118.506) (end 112.8286 118.506) (width 1) (layer "B.Cu") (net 9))
 (segment (start 112.8286 103.6387) (end 112.8286 96.572497) (width 1) (layer "B.Cu") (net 9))
 (segment (start 111.9613 104.506) (end 111.867574 104.506) (width 1) (layer "B.Cu") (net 9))
 (segment (start 117.901097 91.5) (end 165.590811 91.5) (width 1) (layer "B.Cu") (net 9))
 (segment (start 110 106.373574) (end 110 116.105807) (width 1) (layer "B.Cu") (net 9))
 (segment (start 110.703 117.803) (end 110.903034 118.003034) (width 1) (layer "B.Cu") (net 9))
 (arc (start 110 116.105807) (mid 110.182703 117.024321) (end 110.703 117.803) (width 1) (layer "B.Cu") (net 9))
 (arc (start 168.85 92.85) (mid 169.849146 94.345328) (end 170.2 96.109188) (width 1) (layer "B.Cu") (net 9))
 (arc (start 117.901097 91.5) (mid 115.959936 91.88612) (end 114.3143 92.9857) (width 1) (layer "B.Cu") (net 9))
 (arc (start 110.547 105.053) (mid 110.14216 105.658884) (end 110 106.373574) (width 1) (layer "B.Cu") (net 9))
 (arc (start 110.903034 118.003034) (mid 111.460144 118.375283) (end 112.1173 118.506) (width 1) (layer "B.Cu") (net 9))
 (arc (start 114.3143 92.9857) (mid 113.21472 94.631336) (end 112.8286 96.572497) (width 1) (layer "B.Cu") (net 9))
 (arc (start 168.85 92.85) (mid 167.354671 91.850853) (end 165.590811 91.5) (width 1) (layer "B.Cu") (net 9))
 (arc (start 112.8286 103.6387) (mid 112.574573 104.251973) (end 111.9613 104.506) (width 1) (layer "B.Cu") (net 9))
 (arc (start 111.867574 104.506) (mid 111.152884 104.64816) (end 110.547 105.053) (width 1) (layer "B.Cu") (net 9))
 (segment (start 127.2 105.463603) (end 127.2 102) (width 1) (layer "B.Cu") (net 10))
 (segment (start 125.885 110.03) (end 125.3 110.03) (width 1) (layer "B.Cu") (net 10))
 (segment (start 128.1 107.7) (end 128.1 107.636396) (width 1) (layer "B.Cu") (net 10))
 (segment (start 127.605025 108.894974) (end 126.883657 109.616342) (width 1) (layer "B.Cu") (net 10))
 (arc (start 127.65 106.55) (mid 127.983048 107.048442) (end 128.1 107.636396) (width 1) (layer "B.Cu") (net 10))
 (arc (start 128.1 107.7) (mid 127.97136 108.346715) (end 127.605025 108.894974) (width 1) (layer "B.Cu") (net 10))
 (arc (start 126.883657 109.616342) (mid 126.425469 109.922493) (end 125.885 110.03) (width 1) (layer "B.Cu") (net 10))
 (arc (start 127.2 105.463603) (mid 127.316951 106.051556) (end 127.65 106.55) (width 1) (layer "B.Cu") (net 10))
 (segment (start 157.5 113.3625) (end 155.883883 114.978616) (width 1) (layer "B.Cu") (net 13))
 (segment (start 155 117.1125) (end 155 118.3625) (width 1) (layer "B.Cu") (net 13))
 (segment (start 158.225 112.6375) (end 157.5 113.3625) (width 1) (layer "B.Cu") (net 13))
 (segment (start 158.95 108.800609) (end 158.95 110.887195) (width 1) (layer "B.Cu") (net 13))
 (segment (start 162.99 103.85) (end 164.13 103.85) (width 1) (layer "B.Cu") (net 13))
 (segment (start 160.399999 105.299999) (end 161.043898 104.656101) (width 1) (layer "B.Cu") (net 13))
 (arc (start 160.399999 105.299999) (mid 159.326842 106.906092) (end 158.95 108.800609) (width 1) (layer "B.Cu") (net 13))
 (arc (start 162.99 103.85) (mid 161.936777 104.059498) (end 161.043898 104.656101) (width 1) (layer "B.Cu") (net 13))
 (arc (start 155.883883 114.978616) (mid 155.229713 115.95765) (end 155 117.1125) (width 1) (layer "B.Cu") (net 13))
 (arc (start 158.95 110.887195) (mid 158.761578 111.834453) (end 158.225 112.6375) (width 1) (layer "B.Cu") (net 13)))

